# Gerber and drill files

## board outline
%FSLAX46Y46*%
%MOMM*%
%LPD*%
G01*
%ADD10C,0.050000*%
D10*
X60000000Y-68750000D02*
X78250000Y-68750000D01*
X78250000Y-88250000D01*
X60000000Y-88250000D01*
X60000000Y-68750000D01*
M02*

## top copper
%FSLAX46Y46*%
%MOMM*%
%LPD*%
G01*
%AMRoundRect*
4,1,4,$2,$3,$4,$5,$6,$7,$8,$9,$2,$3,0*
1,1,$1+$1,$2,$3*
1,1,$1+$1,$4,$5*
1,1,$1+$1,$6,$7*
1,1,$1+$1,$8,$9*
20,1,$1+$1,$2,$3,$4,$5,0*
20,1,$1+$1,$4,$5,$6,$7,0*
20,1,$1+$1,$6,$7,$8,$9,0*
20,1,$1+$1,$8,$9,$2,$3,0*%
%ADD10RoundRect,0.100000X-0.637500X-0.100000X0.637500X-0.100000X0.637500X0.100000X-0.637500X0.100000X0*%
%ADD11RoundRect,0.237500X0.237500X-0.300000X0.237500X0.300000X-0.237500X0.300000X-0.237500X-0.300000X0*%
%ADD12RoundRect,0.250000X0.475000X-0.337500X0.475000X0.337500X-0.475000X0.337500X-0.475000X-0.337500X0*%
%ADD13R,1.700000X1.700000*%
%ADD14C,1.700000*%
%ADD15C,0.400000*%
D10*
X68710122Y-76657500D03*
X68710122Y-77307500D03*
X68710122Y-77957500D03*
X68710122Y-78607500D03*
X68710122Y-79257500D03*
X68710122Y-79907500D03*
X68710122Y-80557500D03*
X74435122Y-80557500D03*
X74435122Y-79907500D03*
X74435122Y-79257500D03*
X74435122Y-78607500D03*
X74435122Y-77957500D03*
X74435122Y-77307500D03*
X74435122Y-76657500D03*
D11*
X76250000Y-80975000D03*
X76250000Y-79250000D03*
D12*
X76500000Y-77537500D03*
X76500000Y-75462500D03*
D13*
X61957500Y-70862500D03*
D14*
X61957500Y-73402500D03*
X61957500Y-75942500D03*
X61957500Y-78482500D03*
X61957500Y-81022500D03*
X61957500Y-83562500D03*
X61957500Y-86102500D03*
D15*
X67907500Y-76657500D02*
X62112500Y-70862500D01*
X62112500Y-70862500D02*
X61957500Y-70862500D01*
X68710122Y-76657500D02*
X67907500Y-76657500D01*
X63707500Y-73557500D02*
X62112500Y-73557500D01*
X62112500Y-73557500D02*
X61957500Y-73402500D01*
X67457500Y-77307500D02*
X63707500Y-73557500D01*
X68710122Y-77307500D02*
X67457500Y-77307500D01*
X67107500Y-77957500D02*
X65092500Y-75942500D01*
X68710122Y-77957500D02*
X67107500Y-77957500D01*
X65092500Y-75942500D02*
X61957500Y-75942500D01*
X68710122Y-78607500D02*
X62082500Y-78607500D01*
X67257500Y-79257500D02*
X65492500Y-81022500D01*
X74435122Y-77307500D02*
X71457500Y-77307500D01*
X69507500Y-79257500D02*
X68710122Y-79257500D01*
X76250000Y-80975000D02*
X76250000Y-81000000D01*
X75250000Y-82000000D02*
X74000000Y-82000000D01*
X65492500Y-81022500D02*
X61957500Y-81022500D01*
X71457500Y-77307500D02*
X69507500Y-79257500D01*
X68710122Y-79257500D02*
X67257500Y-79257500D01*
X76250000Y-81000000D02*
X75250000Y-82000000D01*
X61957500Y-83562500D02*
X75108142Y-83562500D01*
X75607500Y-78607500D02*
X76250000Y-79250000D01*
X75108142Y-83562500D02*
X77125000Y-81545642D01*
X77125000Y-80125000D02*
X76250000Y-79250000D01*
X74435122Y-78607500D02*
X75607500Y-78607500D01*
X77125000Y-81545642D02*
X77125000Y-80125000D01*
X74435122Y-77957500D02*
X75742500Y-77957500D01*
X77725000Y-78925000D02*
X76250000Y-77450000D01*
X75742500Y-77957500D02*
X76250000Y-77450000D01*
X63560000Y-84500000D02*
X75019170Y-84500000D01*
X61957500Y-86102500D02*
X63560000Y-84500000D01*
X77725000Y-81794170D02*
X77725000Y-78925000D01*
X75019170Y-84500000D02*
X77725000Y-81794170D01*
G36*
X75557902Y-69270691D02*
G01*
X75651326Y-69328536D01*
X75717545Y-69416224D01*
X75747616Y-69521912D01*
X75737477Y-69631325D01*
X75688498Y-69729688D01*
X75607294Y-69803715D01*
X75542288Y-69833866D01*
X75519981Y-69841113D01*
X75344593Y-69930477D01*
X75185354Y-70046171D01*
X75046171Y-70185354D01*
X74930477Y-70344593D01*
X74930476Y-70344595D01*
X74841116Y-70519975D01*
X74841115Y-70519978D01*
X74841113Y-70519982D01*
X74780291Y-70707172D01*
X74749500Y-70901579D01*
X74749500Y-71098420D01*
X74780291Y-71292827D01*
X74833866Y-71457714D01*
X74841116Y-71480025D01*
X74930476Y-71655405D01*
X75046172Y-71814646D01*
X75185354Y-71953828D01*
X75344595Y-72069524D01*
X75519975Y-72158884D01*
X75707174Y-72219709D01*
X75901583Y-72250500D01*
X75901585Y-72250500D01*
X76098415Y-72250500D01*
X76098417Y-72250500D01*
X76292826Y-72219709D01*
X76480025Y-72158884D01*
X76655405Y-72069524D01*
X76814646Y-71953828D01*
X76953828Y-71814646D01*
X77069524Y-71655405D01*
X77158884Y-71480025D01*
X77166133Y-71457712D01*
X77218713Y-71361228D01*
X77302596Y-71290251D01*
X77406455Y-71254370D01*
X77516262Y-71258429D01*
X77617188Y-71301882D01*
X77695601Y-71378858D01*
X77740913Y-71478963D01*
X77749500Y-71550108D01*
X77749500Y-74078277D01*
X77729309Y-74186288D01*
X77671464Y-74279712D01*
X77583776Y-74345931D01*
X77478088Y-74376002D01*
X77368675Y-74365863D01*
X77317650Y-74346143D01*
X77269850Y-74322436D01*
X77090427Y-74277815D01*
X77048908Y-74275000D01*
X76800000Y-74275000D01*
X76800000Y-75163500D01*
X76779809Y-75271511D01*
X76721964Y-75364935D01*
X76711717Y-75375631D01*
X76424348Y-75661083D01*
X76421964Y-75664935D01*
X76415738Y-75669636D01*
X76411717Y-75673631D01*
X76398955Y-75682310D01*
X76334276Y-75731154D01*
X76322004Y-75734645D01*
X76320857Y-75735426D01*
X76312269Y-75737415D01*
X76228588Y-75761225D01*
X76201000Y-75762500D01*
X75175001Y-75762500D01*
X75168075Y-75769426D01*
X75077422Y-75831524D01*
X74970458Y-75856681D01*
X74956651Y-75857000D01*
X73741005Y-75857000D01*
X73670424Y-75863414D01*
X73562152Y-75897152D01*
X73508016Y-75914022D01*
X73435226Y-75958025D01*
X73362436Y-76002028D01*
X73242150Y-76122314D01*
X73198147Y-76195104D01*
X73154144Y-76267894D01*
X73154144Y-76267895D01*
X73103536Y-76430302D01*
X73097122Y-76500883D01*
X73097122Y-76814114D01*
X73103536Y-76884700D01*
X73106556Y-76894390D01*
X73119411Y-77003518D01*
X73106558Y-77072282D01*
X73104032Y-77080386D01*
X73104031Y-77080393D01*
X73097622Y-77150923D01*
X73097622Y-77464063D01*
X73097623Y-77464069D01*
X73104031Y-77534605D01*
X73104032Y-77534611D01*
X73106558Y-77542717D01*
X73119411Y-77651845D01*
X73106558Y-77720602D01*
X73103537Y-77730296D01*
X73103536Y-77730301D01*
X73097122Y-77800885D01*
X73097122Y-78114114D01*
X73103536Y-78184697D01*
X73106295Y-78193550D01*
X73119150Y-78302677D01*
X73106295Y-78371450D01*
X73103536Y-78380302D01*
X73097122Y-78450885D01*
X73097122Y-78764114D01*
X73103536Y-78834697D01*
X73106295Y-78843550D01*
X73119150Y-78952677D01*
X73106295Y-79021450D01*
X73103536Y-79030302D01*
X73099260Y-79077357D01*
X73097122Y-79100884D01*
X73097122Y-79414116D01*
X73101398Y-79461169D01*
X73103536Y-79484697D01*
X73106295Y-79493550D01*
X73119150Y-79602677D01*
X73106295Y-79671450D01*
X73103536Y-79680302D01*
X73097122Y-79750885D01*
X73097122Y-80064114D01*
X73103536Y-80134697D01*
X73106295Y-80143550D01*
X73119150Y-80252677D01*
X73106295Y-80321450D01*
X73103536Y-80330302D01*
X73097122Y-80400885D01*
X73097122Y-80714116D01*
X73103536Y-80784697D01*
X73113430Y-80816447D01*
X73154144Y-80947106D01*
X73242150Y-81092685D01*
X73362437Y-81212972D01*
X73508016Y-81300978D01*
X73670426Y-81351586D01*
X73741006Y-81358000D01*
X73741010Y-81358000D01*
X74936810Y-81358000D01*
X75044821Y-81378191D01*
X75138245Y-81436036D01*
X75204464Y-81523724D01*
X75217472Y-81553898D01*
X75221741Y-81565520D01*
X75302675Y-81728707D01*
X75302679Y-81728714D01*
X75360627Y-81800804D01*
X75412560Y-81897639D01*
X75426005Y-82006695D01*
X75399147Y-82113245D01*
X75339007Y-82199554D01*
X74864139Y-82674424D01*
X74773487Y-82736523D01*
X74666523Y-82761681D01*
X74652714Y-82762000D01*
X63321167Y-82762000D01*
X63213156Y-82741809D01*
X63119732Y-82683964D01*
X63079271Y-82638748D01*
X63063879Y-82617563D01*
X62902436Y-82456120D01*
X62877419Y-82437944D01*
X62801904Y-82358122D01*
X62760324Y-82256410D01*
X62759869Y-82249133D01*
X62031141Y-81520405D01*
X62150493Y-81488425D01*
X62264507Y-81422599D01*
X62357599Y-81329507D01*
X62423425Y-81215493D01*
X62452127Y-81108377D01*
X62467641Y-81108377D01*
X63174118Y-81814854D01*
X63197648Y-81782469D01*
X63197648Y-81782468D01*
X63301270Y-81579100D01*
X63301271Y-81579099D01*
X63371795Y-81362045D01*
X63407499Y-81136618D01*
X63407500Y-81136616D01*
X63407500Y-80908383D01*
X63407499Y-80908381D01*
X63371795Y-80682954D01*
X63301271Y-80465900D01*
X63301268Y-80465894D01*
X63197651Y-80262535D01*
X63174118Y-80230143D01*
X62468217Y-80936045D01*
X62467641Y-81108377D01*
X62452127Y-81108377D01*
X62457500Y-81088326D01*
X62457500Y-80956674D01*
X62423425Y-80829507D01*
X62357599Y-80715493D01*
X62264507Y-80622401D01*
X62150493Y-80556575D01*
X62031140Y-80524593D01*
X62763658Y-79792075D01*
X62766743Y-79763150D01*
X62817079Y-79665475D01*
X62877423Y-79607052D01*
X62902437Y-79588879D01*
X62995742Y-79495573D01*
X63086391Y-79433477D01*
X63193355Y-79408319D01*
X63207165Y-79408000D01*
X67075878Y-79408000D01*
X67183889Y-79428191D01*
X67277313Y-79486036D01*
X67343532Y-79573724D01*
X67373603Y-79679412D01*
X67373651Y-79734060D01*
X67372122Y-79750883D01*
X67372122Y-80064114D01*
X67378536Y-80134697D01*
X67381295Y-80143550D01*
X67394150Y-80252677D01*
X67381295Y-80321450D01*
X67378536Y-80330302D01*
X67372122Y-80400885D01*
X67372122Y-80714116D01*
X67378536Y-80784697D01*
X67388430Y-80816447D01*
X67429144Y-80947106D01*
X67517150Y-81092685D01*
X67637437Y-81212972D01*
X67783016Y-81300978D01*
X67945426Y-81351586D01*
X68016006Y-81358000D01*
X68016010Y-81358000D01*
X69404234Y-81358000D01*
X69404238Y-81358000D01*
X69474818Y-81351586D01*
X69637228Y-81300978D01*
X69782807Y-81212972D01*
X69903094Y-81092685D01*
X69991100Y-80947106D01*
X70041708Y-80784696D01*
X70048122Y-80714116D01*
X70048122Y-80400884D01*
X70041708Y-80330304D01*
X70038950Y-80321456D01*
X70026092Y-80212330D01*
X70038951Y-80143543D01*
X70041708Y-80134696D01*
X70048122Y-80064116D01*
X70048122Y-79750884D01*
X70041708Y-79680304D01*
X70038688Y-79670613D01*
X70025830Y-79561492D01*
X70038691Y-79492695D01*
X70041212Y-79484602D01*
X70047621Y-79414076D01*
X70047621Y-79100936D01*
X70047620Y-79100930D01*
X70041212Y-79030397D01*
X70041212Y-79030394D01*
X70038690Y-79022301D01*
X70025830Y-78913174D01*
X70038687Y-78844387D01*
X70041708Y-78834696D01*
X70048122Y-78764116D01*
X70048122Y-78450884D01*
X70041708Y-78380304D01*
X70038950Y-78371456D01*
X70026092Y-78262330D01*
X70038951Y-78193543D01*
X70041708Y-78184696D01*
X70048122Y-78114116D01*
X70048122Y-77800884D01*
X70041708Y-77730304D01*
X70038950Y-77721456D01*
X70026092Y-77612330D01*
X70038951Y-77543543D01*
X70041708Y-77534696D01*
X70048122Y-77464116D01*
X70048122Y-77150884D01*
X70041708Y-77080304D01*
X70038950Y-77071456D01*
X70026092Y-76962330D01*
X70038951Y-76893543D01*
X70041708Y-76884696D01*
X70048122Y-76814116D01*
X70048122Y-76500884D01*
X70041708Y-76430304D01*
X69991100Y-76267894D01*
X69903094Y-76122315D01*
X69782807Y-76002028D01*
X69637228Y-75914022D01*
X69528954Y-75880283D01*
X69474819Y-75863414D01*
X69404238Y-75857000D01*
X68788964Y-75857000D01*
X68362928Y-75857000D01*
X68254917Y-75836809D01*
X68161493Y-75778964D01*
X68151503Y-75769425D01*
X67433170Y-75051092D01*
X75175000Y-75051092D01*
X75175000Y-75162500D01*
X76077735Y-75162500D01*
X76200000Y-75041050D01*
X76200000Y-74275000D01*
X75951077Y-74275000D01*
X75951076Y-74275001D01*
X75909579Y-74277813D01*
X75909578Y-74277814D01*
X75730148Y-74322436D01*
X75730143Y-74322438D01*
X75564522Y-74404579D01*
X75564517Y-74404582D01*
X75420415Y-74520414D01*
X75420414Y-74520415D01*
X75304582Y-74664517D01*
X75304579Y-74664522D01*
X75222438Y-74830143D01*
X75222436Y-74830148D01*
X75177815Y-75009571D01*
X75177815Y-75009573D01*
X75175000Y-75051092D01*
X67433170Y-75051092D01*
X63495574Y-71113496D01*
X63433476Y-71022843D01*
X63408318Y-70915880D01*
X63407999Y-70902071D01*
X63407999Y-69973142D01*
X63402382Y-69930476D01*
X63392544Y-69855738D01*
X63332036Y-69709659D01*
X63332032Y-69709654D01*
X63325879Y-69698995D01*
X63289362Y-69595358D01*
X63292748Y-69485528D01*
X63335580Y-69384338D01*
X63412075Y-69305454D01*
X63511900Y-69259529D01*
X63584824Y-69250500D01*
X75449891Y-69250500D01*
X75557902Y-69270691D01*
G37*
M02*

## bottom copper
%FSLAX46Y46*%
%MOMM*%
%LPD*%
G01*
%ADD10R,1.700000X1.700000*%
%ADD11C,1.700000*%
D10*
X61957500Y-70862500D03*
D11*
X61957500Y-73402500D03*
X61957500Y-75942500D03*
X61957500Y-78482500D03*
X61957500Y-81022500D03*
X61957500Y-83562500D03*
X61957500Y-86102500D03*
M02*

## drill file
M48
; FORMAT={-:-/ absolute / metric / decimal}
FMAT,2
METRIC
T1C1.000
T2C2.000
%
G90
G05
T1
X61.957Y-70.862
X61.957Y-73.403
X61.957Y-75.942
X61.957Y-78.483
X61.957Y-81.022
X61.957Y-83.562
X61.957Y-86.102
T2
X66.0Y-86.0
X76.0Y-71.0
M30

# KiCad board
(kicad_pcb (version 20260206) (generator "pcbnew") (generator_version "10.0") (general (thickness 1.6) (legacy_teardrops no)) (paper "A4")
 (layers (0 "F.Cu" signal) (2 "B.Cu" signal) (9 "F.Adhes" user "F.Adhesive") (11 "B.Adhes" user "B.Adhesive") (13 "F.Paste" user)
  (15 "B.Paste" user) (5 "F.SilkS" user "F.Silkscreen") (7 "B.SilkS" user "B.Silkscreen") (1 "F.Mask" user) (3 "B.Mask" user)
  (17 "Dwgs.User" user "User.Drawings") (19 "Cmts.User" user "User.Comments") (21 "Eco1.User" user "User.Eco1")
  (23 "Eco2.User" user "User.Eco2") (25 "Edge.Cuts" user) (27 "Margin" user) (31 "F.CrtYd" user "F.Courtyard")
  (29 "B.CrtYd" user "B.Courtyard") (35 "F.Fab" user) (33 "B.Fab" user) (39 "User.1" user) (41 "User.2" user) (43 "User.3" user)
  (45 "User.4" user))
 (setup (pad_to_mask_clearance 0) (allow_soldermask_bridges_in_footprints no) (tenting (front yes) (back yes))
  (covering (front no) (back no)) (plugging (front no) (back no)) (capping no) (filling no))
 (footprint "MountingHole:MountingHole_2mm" (layer "F.Cu") (at 66 86)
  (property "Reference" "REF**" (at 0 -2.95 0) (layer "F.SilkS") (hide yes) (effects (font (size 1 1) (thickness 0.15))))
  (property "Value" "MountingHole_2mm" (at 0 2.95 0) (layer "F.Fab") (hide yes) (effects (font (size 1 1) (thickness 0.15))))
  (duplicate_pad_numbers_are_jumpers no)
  (pad "" np_thru_hole circle (at 0 0) (size 2 2) (drill 2) (layers "*.Cu" "*.Mask")))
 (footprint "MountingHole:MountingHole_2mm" (layer "F.Cu") (at 76 71)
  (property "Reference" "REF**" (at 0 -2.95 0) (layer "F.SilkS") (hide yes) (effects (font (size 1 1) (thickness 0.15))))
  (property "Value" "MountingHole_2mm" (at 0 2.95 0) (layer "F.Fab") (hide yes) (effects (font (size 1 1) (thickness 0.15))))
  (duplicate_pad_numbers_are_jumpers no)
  (pad "" np_thru_hole circle (at 0 0) (size 2 2) (drill 2) (layers "*.Cu" "*.Mask")))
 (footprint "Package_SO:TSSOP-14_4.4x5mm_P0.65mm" (layer "F.Cu") (at 71.572622 78.6075)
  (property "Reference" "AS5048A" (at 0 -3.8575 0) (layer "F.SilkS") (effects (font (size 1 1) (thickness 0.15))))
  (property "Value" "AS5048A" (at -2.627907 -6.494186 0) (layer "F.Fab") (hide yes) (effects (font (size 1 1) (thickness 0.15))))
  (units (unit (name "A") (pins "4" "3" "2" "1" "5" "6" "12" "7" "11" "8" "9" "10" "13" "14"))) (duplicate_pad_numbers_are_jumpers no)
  (pad "1" smd roundrect (at -2.8625 -1.95) (size 1.475 0.4) (layers "F.Cu" "F.Mask" "F.Paste") (roundrect_rratio 0.25) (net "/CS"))
  (pad "2" smd roundrect (at -2.8625 -1.3) (size 1.475 0.4) (layers "F.Cu" "F.Mask" "F.Paste") (roundrect_rratio 0.25) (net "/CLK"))
  (pad "3" smd roundrect (at -2.8625 -0.65) (size 1.475 0.4) (layers "F.Cu" "F.Mask" "F.Paste") (roundrect_rratio 0.25) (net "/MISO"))
  (pad "4" smd roundrect (at -2.8625 0) (size 1.475 0.4) (layers "F.Cu" "F.Mask" "F.Paste") (roundrect_rratio 0.25) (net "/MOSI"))
  (pad "5" smd roundrect (at -2.8625 0.65) (size 1.475 0.4) (layers "F.Cu" "F.Mask" "F.Paste") (roundrect_rratio 0.25) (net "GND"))
  (pad "6" smd roundrect (at -2.8625 1.3) (size 1.475 0.4) (layers "F.Cu" "F.Mask" "F.Paste") (roundrect_rratio 0.25)
   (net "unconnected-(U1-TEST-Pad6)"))
  (pad "7" smd roundrect (at -2.8625 1.95) (size 1.475 0.4) (layers "F.Cu" "F.Mask" "F.Paste") (roundrect_rratio 0.25)
   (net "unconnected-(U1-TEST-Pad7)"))
  (pad "8" smd roundrect (at 2.8625 1.95) (size 1.475 0.4) (layers "F.Cu" "F.Mask" "F.Paste") (roundrect_rratio 0.25)
   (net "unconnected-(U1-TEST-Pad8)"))
  (pad "9" smd roundrect (at 2.8625 1.3) (size 1.475 0.4) (layers "F.Cu" "F.Mask" "F.Paste") (roundrect_rratio 0.25)
   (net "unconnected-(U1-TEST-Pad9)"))
  (pad "10" smd roundrect (at 2.8625 0.65) (size 1.475 0.4) (layers "F.Cu" "F.Mask" "F.Paste") (roundrect_rratio 0.25)
   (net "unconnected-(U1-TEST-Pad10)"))
  (pad "11" smd roundrect (at 2.8625 0) (size 1.475 0.4) (layers "F.Cu" "F.Mask" "F.Paste") (roundrect_rratio 0.25) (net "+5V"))
  (pad "12" smd roundrect (at 2.8625 -0.65) (size 1.475 0.4) (layers "F.Cu" "F.Mask" "F.Paste") (roundrect_rratio 0.25) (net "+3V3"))
  (pad "13" smd roundrect (at 2.8625 -1.3) (size 1.475 0.4) (layers "F.Cu" "F.Mask" "F.Paste") (roundrect_rratio 0.25) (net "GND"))
  (pad "14" smd roundrect (at 2.8625 -1.95) (size 1.475 0.4) (layers "F.Cu" "F.Mask" "F.Paste") (roundrect_rratio 0.25)
   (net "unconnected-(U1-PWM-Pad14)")))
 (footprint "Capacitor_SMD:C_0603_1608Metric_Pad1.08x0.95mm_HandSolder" (layer "F.Cu") (at 76.25 80.1125 90)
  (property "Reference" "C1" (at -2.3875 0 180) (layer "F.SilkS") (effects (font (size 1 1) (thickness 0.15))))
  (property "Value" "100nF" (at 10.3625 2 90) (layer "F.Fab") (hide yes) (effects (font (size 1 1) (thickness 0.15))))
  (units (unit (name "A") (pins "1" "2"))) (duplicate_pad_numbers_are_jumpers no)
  (pad "1" smd roundrect (at -0.8625 0 90) (size 1.075 0.95) (layers "F.Cu" "F.Mask" "F.Paste") (roundrect_rratio 0.25) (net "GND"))
  (pad "2" smd roundrect (at 0.8625 0 90) (size 1.075 0.95) (layers "F.Cu" "F.Mask" "F.Paste") (roundrect_rratio 0.25) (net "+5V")))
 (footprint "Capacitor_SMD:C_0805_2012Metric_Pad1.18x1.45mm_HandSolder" (layer "F.Cu") (at 76.5 76.5 90)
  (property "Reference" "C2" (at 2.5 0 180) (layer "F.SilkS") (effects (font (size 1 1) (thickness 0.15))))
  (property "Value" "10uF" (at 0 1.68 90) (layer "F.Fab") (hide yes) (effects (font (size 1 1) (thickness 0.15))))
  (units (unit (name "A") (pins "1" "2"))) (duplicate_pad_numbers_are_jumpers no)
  (pad "1" smd roundrect (at -1.0375 0 90) (size 1.175 1.45) (layers "F.Cu" "F.Mask" "F.Paste") (roundrect_rratio 0.212766) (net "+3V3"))
  (pad "2" smd roundrect (at 1.0375 0 90) (size 1.175 1.45) (layers "F.Cu" "F.Mask" "F.Paste") (roundrect_rratio 0.212766) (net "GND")))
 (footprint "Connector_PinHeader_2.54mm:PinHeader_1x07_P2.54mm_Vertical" (layer "F.Cu") (at 61.9575 70.8625)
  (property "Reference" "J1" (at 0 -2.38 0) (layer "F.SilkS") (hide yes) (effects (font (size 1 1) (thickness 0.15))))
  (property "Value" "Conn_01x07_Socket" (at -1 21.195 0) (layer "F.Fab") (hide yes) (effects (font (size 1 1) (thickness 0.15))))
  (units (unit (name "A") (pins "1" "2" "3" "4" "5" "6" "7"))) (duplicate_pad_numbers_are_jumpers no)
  (pad "1" thru_hole rect (at 0 0) (size 1.7 1.7) (drill 1) (layers "*.Cu" "*.Mask") (remove_unused_layers no) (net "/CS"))
  (pad "2" thru_hole circle (at 0 2.54) (size 1.7 1.7) (drill 1) (layers "*.Cu" "*.Mask") (remove_unused_layers no) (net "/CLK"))
  (pad "3" thru_hole circle (at 0 5.08) (size 1.7 1.7) (drill 1) (layers "*.Cu" "*.Mask") (remove_unused_layers no) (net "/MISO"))
  (pad "4" thru_hole circle (at 0 7.62) (size 1.7 1.7) (drill 1) (layers "*.Cu" "*.Mask") (remove_unused_layers no) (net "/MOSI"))
  (pad "5" thru_hole circle (at 0 10.16) (size 1.7 1.7) (drill 1) (layers "*.Cu" "*.Mask") (remove_unused_layers no) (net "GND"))
  (pad "6" thru_hole circle (at 0 12.7) (size 1.7 1.7) (drill 1) (layers "*.Cu" "*.Mask") (remove_unused_layers no) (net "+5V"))
  (pad "7" thru_hole circle (at 0 15.24) (size 1.7 1.7) (drill 1) (layers "*.Cu" "*.Mask") (remove_unused_layers no) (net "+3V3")))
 (gr_rect (start 60 68.75) (end 78.25 88.25) (stroke (width 0.05) (type default)) (fill no) (layer "Edge.Cuts"))
 (segment (start 67.9075 76.6575) (end 62.1125 70.8625) (width 0.4) (layer "F.Cu") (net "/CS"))
 (segment (start 62.1125 70.8625) (end 61.9575 70.8625) (width 0.4) (layer "F.Cu") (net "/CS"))
 (segment (start 68.710122 76.6575) (end 67.9075 76.6575) (width 0.4) (layer "F.Cu") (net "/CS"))
 (segment (start 63.7075 73.5575) (end 62.1125 73.5575) (width 0.4) (layer "F.Cu") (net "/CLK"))
 (segment (start 62.1125 73.5575) (end 61.9575 73.4025) (width 0.4) (layer "F.Cu") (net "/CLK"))
 (segment (start 67.4575 77.3075) (end 63.7075 73.5575) (width 0.4) (layer "F.Cu") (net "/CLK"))
 (segment (start 68.710122 77.3075) (end 67.4575 77.3075) (width 0.4) (layer "F.Cu") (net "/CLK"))
 (segment (start 67.1075 77.9575) (end 65.0925 75.9425) (width 0.4) (layer "F.Cu") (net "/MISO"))
 (segment (start 68.710122 77.9575) (end 67.1075 77.9575) (width 0.4) (layer "F.Cu") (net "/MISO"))
 (segment (start 65.0925 75.9425) (end 61.9575 75.9425) (width 0.4) (layer "F.Cu") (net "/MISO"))
 (segment (start 68.710122 78.6075) (end 62.0825 78.6075) (width 0.4) (layer "F.Cu") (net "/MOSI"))
 (segment (start 67.2575 79.2575) (end 65.4925 81.0225) (width 0.4) (layer "F.Cu") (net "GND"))
 (segment (start 74.435122 77.3075) (end 71.4575 77.3075) (width 0.4) (layer "F.Cu") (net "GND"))
 (segment (start 69.5075 79.2575) (end 68.710122 79.2575) (width 0.4) (layer "F.Cu") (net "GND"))
 (segment (start 76.25 80.975) (end 76.25 81) (width 0.4) (layer "F.Cu") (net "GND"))
 (segment (start 75.25 82) (end 74 82) (width 0.4) (layer "F.Cu") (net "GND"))
 (segment (start 65.4925 81.0225) (end 61.9575 81.0225) (width 0.4) (layer "F.Cu") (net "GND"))
 (segment (start 71.4575 77.3075) (end 69.5075 79.2575) (width 0.4) (layer "F.Cu") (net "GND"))
 (segment (start 68.710122 79.2575) (end 67.2575 79.2575) (width 0.4) (layer "F.Cu") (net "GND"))
 (segment (start 76.25 81) (end 75.25 82) (width 0.4) (layer "F.Cu") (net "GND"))
 (segment (start 61.9575 83.5625) (end 75.108142 83.5625) (width 0.4) (layer "F.Cu") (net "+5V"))
 (segment (start 75.6075 78.6075) (end 76.25 79.25) (width 0.4) (layer "F.Cu") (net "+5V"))
 (segment (start 75.108142 83.5625) (end 77.125 81.545642) (width 0.4) (layer "F.Cu") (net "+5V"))
 (segment (start 77.125 80.125) (end 76.25 79.25) (width 0.4) (layer "F.Cu") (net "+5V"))
 (segment (start 74.435122 78.6075) (end 75.6075 78.6075) (width 0.4) (layer "F.Cu") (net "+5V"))
 (segment (start 77.125 81.545642) (end 77.125 80.125) (width 0.4) (layer "F.Cu") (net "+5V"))
 (segment (start 74.435122 77.9575) (end 75.7425 77.9575) (width 0.4) (layer "F.Cu") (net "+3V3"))
 (segment (start 77.725 78.925) (end 76.25 77.45) (width 0.4) (layer "F.Cu") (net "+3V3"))
 (segment (start 75.7425 77.9575) (end 76.25 77.45) (width 0.4) (layer "F.Cu") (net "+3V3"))
 (segment (start 63.56 84.5) (end 75.01917 84.5) (width 0.4) (layer "F.Cu") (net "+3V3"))
 (segment (start 61.9575 86.1025) (end 63.56 84.5) (width 0.4) (layer "F.Cu") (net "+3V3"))
 (segment (start 77.725 81.79417) (end 77.725 78.925) (width 0.4) (layer "F.Cu") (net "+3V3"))
 (segment (start 75.01917 84.5) (end 77.725 81.79417) (width 0.4) (layer "F.Cu") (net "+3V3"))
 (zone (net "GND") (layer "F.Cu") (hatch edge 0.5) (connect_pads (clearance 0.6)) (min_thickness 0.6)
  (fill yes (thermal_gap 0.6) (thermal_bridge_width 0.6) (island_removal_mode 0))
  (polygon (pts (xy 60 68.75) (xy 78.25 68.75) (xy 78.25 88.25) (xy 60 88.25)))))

